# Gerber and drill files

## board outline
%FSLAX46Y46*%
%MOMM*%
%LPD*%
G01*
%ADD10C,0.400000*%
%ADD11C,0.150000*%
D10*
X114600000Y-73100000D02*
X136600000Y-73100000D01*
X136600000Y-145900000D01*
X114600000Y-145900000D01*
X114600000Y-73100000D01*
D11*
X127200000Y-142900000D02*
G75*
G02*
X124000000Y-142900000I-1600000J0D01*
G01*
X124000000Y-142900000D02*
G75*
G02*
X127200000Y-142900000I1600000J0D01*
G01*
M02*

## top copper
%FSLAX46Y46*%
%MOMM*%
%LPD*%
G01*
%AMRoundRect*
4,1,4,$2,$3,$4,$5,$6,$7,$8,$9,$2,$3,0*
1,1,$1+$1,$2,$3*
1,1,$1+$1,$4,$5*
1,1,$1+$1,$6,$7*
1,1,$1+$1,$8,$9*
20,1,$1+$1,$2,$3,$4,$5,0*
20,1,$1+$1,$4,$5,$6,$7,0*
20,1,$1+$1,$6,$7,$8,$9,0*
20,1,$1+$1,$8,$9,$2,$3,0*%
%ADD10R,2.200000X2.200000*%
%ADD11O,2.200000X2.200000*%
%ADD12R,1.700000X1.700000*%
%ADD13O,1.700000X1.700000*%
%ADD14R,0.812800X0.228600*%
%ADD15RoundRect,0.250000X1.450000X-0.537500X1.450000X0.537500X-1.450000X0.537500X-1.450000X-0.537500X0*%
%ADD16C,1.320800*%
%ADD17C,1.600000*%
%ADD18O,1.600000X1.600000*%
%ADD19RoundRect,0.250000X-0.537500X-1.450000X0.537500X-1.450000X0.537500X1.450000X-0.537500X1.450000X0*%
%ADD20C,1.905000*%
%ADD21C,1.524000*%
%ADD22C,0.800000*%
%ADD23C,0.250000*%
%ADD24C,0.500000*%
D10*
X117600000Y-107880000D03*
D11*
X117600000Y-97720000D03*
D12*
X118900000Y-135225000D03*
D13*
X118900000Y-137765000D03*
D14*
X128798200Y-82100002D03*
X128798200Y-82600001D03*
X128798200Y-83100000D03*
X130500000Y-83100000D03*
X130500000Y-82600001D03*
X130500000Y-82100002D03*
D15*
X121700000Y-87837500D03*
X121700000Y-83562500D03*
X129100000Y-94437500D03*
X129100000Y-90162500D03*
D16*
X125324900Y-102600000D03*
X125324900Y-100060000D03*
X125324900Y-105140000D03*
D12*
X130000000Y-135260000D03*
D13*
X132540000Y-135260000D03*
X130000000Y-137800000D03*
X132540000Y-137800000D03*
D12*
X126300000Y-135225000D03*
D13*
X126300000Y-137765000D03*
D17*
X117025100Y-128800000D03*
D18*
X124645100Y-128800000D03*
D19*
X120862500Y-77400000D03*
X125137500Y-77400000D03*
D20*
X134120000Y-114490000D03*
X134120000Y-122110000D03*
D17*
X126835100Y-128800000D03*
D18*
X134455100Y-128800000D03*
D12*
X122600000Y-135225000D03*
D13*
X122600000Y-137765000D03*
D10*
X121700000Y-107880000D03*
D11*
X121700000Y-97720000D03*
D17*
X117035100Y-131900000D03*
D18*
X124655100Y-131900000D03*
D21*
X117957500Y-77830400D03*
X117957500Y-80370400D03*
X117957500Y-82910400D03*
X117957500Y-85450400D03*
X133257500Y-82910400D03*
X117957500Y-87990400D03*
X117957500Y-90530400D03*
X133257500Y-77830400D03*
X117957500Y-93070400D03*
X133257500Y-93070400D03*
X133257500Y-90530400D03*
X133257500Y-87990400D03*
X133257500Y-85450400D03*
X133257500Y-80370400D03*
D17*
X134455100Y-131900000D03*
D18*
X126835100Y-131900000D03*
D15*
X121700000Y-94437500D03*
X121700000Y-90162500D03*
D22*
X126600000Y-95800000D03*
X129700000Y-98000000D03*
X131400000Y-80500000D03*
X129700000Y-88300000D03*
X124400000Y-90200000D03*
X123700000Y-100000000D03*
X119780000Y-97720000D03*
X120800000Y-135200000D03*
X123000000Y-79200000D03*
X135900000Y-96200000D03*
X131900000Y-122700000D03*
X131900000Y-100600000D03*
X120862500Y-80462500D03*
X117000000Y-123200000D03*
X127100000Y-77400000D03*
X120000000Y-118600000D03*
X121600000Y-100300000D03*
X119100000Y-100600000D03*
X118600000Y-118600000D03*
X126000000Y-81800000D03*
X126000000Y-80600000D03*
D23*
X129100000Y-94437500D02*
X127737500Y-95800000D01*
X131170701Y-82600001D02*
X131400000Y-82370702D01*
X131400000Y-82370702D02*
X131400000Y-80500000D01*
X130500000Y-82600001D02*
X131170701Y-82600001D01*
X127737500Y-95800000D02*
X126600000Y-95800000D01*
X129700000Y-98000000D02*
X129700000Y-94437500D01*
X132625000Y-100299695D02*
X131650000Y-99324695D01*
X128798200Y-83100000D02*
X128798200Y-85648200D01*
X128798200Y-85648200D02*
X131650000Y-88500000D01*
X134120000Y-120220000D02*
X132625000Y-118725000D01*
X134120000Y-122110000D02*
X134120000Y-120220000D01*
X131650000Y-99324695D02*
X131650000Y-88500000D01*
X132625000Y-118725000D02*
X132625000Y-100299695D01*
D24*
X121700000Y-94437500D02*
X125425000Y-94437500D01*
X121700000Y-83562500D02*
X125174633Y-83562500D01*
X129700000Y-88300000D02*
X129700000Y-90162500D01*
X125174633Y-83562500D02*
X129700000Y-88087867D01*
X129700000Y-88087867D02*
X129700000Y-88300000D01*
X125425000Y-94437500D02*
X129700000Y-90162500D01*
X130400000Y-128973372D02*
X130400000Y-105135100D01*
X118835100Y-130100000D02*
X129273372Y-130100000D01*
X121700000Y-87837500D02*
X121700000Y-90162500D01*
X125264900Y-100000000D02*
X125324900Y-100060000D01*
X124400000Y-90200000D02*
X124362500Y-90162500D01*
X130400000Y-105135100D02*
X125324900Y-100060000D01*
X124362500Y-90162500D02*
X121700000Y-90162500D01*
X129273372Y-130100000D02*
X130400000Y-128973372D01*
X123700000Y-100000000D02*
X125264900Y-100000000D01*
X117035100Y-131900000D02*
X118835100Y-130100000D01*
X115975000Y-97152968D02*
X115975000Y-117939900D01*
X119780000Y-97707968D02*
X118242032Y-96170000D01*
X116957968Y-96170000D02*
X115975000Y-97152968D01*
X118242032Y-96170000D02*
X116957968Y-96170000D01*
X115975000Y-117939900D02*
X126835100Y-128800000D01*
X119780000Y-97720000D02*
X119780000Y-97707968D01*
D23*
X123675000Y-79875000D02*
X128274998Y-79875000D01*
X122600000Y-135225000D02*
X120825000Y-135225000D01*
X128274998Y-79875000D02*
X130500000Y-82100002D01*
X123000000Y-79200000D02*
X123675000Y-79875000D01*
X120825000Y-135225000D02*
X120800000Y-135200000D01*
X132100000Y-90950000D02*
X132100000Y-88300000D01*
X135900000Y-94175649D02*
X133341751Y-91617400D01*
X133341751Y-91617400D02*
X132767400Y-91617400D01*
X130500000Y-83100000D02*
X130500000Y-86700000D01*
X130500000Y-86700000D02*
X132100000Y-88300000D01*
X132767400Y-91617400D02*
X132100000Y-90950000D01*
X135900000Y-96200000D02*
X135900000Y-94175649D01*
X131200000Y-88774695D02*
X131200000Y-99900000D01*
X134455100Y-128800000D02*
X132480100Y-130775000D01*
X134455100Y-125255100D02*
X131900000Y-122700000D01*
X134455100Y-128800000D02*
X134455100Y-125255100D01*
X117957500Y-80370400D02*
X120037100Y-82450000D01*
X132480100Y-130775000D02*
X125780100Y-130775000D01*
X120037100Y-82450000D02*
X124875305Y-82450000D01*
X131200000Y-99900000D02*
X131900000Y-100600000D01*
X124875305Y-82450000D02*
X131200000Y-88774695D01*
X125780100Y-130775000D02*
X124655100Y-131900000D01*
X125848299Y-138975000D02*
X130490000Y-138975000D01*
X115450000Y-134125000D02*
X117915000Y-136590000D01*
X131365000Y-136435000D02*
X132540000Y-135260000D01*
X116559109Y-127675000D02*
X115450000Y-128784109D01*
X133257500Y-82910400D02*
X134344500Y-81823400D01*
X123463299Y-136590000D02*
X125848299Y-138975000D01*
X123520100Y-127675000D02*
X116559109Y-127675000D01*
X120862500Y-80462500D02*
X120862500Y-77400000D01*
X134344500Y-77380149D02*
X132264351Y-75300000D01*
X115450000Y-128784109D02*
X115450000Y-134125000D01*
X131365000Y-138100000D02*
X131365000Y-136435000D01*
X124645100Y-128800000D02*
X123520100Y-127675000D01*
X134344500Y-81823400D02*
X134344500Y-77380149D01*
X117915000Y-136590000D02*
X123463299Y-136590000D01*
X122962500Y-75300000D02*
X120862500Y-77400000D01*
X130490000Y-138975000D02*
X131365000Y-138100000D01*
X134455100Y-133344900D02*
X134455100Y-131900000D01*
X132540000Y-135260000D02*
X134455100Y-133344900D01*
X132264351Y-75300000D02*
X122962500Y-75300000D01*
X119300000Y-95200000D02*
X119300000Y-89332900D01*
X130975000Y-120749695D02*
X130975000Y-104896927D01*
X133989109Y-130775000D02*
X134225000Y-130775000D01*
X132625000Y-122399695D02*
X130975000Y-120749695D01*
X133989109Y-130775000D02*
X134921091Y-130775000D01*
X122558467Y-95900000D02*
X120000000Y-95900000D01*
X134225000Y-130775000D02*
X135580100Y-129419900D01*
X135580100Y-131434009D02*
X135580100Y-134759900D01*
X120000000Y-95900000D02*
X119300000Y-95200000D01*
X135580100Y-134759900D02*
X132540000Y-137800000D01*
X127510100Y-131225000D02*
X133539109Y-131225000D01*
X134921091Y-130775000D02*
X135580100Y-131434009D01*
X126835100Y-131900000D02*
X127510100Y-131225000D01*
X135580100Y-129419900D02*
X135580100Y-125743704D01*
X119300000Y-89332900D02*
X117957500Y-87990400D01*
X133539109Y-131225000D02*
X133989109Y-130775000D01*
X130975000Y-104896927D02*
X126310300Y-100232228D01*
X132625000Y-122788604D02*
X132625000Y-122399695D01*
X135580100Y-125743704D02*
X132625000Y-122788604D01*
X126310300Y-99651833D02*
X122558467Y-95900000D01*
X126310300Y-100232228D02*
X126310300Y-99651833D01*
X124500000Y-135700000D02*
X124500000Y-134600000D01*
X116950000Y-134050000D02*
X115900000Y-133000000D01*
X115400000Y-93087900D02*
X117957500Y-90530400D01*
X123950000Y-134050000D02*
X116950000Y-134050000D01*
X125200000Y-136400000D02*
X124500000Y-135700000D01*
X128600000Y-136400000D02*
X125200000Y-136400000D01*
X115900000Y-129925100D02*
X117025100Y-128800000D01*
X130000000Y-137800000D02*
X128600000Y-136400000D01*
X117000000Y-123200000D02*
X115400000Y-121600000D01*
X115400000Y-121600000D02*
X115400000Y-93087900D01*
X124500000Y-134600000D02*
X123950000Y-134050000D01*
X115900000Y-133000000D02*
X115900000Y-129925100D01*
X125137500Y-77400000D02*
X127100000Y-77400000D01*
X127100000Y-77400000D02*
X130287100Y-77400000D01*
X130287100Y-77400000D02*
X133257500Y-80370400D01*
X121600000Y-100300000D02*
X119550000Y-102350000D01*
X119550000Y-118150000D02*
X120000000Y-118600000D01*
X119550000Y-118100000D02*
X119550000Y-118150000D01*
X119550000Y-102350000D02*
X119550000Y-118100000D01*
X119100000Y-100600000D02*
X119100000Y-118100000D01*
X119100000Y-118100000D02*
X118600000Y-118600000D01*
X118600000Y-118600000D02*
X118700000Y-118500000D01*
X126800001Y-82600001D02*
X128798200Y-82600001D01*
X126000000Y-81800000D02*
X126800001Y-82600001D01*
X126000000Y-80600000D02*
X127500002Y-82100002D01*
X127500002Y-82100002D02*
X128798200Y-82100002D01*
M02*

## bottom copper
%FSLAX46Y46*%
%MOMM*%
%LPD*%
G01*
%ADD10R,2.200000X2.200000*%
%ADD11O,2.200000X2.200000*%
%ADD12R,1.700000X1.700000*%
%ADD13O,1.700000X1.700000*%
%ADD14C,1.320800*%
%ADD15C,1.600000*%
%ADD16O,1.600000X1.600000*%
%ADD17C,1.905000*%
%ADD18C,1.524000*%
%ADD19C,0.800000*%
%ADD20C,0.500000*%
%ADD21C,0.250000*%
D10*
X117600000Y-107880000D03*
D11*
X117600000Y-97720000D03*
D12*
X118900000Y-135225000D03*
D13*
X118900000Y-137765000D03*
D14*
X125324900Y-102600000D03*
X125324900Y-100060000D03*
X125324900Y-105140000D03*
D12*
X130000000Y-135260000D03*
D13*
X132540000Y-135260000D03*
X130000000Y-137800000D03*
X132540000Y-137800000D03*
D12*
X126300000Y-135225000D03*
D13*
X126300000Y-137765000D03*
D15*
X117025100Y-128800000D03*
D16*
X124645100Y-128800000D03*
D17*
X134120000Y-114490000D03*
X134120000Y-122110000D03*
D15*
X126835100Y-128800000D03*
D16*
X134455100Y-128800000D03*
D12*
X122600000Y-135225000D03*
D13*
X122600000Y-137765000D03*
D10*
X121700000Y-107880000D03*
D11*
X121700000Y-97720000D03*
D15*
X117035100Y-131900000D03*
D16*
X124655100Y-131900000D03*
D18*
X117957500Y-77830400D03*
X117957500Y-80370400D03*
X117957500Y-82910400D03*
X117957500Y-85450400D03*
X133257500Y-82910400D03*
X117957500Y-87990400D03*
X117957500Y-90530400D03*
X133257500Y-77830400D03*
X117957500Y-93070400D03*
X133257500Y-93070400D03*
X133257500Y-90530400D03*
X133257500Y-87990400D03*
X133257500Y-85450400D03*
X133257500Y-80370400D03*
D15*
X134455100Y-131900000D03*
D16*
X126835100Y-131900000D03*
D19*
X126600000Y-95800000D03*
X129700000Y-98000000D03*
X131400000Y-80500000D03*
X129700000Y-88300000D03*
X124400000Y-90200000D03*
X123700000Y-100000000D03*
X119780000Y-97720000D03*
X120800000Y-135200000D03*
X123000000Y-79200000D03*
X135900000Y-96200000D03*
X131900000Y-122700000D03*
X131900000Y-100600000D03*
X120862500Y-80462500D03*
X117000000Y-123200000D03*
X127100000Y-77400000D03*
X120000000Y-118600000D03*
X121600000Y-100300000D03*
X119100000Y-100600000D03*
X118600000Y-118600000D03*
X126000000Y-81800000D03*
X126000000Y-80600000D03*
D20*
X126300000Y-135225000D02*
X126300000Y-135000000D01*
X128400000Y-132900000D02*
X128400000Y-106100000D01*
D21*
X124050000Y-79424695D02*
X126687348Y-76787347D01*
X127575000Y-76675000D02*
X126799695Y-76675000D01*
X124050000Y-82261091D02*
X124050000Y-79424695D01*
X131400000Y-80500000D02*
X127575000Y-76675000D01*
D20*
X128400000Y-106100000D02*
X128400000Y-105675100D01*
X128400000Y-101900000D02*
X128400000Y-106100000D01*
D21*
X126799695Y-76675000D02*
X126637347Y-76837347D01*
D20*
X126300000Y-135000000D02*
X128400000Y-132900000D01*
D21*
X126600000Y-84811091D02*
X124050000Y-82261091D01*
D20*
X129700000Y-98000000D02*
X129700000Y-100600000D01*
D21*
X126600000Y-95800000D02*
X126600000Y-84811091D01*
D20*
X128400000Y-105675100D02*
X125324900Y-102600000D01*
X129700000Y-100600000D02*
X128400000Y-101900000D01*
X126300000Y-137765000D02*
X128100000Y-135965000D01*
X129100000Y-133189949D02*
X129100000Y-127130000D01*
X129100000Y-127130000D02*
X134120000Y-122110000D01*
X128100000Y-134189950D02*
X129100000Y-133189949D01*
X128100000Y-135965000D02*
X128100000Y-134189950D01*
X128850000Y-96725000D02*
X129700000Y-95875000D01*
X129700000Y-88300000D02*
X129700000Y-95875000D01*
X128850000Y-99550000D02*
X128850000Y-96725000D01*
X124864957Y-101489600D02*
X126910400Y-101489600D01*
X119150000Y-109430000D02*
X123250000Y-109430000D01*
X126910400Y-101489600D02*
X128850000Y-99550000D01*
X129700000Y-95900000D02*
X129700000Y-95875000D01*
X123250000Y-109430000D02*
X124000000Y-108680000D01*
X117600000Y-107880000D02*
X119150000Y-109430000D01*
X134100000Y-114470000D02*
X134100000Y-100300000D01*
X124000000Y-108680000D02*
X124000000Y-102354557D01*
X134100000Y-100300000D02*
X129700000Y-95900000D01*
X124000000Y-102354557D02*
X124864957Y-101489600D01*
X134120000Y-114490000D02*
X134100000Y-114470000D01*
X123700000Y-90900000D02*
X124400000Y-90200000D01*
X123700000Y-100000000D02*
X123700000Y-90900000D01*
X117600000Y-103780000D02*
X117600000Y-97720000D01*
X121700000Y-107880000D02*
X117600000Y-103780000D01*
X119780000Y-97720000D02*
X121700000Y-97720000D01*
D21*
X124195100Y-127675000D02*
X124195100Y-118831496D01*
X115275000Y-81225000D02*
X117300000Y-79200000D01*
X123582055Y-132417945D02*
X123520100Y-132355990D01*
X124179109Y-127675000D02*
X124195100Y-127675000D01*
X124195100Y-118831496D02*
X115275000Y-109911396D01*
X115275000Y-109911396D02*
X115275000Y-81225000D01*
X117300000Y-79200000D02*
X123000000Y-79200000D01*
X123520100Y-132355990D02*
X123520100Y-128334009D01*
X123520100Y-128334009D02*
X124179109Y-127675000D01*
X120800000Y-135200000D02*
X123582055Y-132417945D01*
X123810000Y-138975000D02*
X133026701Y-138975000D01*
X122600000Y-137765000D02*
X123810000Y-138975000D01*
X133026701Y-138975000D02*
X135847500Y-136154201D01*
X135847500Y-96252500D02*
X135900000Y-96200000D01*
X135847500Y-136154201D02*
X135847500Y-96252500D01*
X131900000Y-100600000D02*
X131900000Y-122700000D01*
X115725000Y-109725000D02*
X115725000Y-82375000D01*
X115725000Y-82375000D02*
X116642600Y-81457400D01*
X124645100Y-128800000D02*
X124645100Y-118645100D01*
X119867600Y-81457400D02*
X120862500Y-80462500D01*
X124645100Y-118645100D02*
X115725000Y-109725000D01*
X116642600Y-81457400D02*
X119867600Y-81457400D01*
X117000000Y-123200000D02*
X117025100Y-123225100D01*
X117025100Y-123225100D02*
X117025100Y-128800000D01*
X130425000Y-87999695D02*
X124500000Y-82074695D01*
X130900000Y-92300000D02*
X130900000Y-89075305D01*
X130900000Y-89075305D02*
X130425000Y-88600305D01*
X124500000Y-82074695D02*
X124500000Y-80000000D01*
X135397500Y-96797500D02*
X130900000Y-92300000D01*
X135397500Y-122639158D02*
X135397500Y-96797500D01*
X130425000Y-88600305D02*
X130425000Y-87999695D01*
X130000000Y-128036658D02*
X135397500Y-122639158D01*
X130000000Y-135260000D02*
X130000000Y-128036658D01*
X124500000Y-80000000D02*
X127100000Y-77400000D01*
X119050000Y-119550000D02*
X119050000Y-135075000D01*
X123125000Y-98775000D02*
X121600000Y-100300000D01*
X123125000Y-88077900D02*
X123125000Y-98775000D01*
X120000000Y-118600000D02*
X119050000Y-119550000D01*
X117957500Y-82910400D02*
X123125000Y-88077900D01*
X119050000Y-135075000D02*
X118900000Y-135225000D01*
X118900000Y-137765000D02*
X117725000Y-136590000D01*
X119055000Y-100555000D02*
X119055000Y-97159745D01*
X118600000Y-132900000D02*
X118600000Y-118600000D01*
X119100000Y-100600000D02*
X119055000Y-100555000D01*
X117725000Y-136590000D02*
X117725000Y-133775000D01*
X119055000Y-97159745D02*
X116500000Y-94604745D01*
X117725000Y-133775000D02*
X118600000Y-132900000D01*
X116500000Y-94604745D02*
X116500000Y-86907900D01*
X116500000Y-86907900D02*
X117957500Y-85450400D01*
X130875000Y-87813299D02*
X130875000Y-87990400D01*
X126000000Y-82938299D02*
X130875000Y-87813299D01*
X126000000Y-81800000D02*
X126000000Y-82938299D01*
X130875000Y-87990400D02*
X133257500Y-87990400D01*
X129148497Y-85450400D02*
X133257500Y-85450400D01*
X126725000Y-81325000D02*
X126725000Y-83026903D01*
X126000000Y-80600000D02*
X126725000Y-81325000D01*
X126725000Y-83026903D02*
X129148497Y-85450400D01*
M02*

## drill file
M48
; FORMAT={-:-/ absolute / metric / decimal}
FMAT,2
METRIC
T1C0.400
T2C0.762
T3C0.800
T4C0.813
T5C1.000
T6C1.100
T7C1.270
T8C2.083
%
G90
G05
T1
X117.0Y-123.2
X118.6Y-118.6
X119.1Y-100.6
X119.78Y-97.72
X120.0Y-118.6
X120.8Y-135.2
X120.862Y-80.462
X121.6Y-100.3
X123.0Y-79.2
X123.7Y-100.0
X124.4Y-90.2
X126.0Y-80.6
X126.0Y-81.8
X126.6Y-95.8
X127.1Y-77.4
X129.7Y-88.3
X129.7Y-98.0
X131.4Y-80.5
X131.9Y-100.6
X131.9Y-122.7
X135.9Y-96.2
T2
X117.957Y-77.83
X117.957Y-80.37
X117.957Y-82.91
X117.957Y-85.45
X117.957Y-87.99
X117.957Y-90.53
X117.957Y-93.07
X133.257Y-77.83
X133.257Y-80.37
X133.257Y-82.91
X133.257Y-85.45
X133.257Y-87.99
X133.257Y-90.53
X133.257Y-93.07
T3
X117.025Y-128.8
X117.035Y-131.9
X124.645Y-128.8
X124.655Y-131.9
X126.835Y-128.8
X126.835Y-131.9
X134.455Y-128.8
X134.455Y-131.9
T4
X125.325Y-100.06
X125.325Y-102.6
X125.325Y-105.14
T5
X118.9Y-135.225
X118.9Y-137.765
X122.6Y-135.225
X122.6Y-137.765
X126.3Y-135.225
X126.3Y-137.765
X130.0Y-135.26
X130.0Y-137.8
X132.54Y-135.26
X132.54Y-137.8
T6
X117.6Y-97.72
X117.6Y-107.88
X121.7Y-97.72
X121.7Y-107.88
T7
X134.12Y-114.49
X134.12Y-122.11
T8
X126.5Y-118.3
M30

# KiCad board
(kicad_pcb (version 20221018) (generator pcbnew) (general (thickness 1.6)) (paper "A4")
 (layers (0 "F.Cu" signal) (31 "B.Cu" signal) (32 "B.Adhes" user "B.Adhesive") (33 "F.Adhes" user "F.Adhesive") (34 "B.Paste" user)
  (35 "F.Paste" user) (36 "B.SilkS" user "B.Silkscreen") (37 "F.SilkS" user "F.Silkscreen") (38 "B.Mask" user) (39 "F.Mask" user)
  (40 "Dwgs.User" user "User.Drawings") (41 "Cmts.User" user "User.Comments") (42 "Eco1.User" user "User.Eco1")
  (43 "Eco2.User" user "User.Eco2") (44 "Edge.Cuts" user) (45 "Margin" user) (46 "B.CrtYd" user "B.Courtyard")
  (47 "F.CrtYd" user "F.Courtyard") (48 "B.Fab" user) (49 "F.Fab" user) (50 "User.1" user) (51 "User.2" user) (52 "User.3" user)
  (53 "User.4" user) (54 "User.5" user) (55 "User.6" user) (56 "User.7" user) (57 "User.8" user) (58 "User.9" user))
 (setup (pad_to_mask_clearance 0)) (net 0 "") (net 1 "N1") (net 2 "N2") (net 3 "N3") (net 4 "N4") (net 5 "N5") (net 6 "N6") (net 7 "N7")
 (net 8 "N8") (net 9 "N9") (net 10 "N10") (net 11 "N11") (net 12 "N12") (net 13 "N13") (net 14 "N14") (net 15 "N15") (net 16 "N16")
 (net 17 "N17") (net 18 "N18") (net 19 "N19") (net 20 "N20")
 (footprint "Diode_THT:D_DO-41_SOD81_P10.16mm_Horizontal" (layer "F.Cu") (at 117.6 107.88 90)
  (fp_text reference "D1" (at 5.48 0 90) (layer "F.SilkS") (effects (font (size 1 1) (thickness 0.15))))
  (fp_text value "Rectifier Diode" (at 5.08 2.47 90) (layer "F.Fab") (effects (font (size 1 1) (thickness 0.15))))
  (pad "1" thru_hole rect (at 0 0 90) (size 2.2 2.2) (drill 1.1) (layers "*.Cu" "*.Mask") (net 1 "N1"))
  (pad "2" thru_hole oval (at 10.16 0 90) (size 2.2 2.2) (drill 1.1) (layers "*.Cu" "*.Mask") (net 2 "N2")))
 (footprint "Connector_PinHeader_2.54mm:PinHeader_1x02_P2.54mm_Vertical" (layer "F.Cu") (at 118.9 135.225)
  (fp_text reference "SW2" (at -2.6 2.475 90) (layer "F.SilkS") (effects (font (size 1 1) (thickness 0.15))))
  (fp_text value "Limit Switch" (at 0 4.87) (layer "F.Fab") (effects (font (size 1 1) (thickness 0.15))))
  (pad "1" thru_hole rect (at 0 0) (size 1.7 1.7) (drill 1) (layers "*.Cu" "*.Mask") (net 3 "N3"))
  (pad "2" thru_hole oval (at 0 2.54) (size 1.7 1.7) (drill 1) (layers "*.Cu" "*.Mask") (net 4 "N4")))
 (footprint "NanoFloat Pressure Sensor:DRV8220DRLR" (layer "F.Cu") (at 129.6491 82.600001)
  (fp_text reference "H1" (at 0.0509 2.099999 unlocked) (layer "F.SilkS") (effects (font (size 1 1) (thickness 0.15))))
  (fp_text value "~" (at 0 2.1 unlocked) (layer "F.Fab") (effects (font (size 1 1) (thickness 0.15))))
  (pad "1" smd rect (at -0.8509 -0.499999) (size 0.8128 0.2286) (layers "F.Cu" "F.Paste" "F.Mask") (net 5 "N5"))
  (pad "2" smd rect (at -0.8509 0) (size 0.8128 0.2286) (layers "F.Cu" "F.Paste" "F.Mask") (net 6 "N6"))
  (pad "3" smd rect (at -0.8509 0.499999) (size 0.8128 0.2286) (layers "F.Cu" "F.Paste" "F.Mask") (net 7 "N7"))
  (pad "4" smd rect (at 0.8509 0.499999) (size 0.8128 0.2286) (layers "F.Cu" "F.Paste" "F.Mask") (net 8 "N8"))
  (pad "5" smd rect (at 0.8509 0) (size 0.8128 0.2286) (layers "F.Cu" "F.Paste" "F.Mask") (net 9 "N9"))
  (pad "6" smd rect (at 0.8509 -0.499999) (size 0.8128 0.2286) (layers "F.Cu" "F.Paste" "F.Mask") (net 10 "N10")))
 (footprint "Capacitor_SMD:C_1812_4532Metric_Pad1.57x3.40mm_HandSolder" (layer "F.Cu") (at 121.7 85.7 90)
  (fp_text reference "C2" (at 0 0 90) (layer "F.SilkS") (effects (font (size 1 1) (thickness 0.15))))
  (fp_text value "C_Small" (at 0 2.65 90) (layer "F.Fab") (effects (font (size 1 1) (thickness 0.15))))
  (pad "1" smd roundrect (at -2.1375 0 90) (size 1.575 3.4) (layers "F.Cu" "F.Paste" "F.Mask") (roundrect_rratio 0.1587301587)
   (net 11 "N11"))
  (pad "2" smd roundrect (at 2.1375 0 90) (size 1.575 3.4) (layers "F.Cu" "F.Paste" "F.Mask") (roundrect_rratio 0.1587301587) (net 1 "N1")))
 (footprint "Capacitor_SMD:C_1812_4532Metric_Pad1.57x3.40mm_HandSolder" (layer "F.Cu") (at 129.1 92.3 90)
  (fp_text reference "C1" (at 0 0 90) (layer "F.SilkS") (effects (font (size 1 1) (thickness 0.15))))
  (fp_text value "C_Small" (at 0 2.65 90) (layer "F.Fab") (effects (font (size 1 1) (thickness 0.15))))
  (pad "1" smd roundrect (at -2.1375 0 90) (size 1.575 3.4) (layers "F.Cu" "F.Paste" "F.Mask") (roundrect_rratio 0.1587301587) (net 9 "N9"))
  (pad "2" smd roundrect (at 2.1375 0 90) (size 1.575 3.4) (layers "F.Cu" "F.Paste" "F.Mask") (roundrect_rratio 0.1587301587) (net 1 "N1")))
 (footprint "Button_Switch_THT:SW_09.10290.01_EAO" (layer "F.Cu") (at 125.3249 102.6 90)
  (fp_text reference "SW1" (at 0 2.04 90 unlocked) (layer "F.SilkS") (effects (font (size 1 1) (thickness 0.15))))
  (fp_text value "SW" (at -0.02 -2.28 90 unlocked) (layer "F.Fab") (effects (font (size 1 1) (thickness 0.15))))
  (pad "1" thru_hole circle (at 0 0 90) (size 1.3208 1.3208) (drill 0.8128) (layers "*.Cu" "*.Mask") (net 9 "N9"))
  (pad "2" thru_hole circle (at 2.54 0 90) (size 1.3208 1.3208) (drill 0.8128) (layers "*.Cu" "*.Mask") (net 11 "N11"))
  (pad "3" thru_hole circle (at -2.54 0 90) (size 1.3208 1.3208) (drill 0.8128) (layers "*.Cu" "*.Mask") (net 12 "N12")))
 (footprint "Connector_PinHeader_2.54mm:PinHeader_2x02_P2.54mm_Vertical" (layer "F.Cu") (at 130 135.26)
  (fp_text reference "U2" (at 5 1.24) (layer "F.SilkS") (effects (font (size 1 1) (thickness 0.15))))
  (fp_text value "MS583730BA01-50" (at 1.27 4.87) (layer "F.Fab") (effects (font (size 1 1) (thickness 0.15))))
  (pad "1" thru_hole rect (at 0 0) (size 1.7 1.7) (drill 1) (layers "*.Cu" "*.Mask") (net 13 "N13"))
  (pad "2" thru_hole oval (at 2.54 0) (size 1.7 1.7) (drill 1) (layers "*.Cu" "*.Mask") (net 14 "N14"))
  (pad "3" thru_hole oval (at 0 2.54) (size 1.7 1.7) (drill 1) (layers "*.Cu" "*.Mask") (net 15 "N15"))
  (pad "4" thru_hole oval (at 2.54 2.54) (size 1.7 1.7) (drill 1) (layers "*.Cu" "*.Mask") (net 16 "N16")))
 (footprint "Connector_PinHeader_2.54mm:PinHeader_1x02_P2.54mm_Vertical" (layer "F.Cu") (at 126.3 135.225)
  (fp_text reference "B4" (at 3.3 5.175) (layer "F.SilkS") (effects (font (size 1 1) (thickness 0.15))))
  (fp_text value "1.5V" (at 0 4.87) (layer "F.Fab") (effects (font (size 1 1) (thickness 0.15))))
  (pad "1" thru_hole rect (at 0 0) (size 1.7 1.7) (drill 1) (layers "*.Cu" "*.Mask") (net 9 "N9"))
  (pad "2" thru_hole oval (at 0 2.54) (size 1.7 1.7) (drill 1) (layers "*.Cu" "*.Mask") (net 7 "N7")))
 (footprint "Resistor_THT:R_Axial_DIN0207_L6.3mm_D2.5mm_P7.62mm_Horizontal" (layer "F.Cu") (at 117.0251 128.8)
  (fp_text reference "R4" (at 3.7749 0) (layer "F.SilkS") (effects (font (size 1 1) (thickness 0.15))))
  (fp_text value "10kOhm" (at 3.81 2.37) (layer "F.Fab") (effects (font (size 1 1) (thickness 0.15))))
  (pad "1" thru_hole circle (at 0 0) (size 1.6 1.6) (drill 0.8) (layers "*.Cu" "*.Mask") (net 15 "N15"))
  (pad "2" thru_hole oval (at 7.62 0) (size 1.6 1.6) (drill 0.8) (layers "*.Cu" "*.Mask") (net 14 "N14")))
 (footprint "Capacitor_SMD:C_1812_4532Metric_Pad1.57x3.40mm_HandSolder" (layer "F.Cu") (at 123 77.4)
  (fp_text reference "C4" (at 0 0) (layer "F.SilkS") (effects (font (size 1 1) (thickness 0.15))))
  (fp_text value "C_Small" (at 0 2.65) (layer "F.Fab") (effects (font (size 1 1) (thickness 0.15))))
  (pad "1" smd roundrect (at -2.1375 0) (size 1.575 3.4) (layers "F.Cu" "F.Paste" "F.Mask") (roundrect_rratio 0.1587301587) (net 14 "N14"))
  (pad "2" smd roundrect (at 2.1375 0) (size 1.575 3.4) (layers "F.Cu" "F.Paste" "F.Mask") (roundrect_rratio 0.1587301587) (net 13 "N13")))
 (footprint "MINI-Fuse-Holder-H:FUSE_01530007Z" (layer "F.Cu") (at 126.5 118.3 -90)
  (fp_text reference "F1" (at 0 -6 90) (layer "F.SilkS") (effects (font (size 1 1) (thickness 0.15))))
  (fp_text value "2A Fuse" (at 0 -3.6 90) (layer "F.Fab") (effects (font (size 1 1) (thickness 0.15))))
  (pad "" np_thru_hole circle (at 0 0 270) (size 2.0828 2.0828) (drill 2.0828) (layers "*.Cu" "*.Mask"))
  (pad "1" thru_hole circle (at -3.81 -7.62 270) (size 1.905 1.905) (drill 1.27) (layers "*.Cu" "*.Mask") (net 1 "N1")
   (solder_mask_margin 0.102))
  (pad "2" thru_hole circle (at 3.81 -7.62 270) (size 1.905 1.905) (drill 1.27) (layers "*.Cu" "*.Mask") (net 7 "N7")
   (solder_mask_margin 0.102)))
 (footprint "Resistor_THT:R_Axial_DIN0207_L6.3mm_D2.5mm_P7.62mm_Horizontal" (layer "F.Cu") (at 126.8351 128.8)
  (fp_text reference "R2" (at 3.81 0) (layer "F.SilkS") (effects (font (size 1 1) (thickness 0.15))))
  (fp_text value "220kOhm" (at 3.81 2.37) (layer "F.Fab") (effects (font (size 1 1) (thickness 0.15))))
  (pad "1" thru_hole circle (at 0 0) (size 1.6 1.6) (drill 0.8) (layers "*.Cu" "*.Mask") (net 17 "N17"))
  (pad "2" thru_hole oval (at 7.62 0) (size 1.6 1.6) (drill 0.8) (layers "*.Cu" "*.Mask") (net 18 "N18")))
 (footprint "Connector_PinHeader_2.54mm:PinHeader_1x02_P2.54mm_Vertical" (layer "F.Cu") (at 122.6 135.225)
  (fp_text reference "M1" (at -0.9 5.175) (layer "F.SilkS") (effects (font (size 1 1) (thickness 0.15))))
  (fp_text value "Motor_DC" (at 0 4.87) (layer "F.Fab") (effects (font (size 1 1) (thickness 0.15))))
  (pad "1" thru_hole rect (at 0 0) (size 1.7 1.7) (drill 1) (layers "*.Cu" "*.Mask") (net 10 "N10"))
  (pad "2" thru_hole oval (at 0 2.54) (size 1.7 1.7) (drill 1) (layers "*.Cu" "*.Mask") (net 8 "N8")))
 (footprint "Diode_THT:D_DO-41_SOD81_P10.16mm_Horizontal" (layer "F.Cu") (at 121.7 107.88 90)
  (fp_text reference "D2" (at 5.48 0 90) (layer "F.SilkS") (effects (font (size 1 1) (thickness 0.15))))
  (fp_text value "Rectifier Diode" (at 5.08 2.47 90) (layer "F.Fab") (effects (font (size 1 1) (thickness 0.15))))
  (pad "1" thru_hole rect (at 0 0 90) (size 2.2 2.2) (drill 1.1) (layers "*.Cu" "*.Mask") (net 2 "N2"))
  (pad "2" thru_hole oval (at 10.16 0 90) (size 2.2 2.2) (drill 1.1) (layers "*.Cu" "*.Mask") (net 17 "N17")))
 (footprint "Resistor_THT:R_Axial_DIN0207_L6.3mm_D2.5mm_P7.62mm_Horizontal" (layer "F.Cu") (at 117.0351 131.9)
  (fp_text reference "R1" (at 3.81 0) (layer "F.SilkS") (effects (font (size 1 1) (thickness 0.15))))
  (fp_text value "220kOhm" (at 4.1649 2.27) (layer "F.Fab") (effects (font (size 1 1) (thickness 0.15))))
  (pad "1" thru_hole circle (at 0 0) (size 1.6 1.6) (drill 0.8) (layers "*.Cu" "*.Mask") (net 11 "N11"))
  (pad "2" thru_hole oval (at 7.62 0) (size 1.6 1.6) (drill 0.8) (layers "*.Cu" "*.Mask") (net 18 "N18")))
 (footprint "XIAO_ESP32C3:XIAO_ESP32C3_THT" (layer "F.Cu") (at 125.5575 87.8704)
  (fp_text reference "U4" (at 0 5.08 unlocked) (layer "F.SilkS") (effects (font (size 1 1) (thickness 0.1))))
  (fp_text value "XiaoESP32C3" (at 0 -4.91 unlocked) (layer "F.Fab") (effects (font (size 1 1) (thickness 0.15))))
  (pad "0" thru_hole circle (at -7.6 -10.04) (size 1.524 1.524) (drill 0.762) (layers "*.Cu" "*.Mask"))
  (pad "1" thru_hole circle (at -7.6 -7.5) (size 1.524 1.524) (drill 0.762) (layers "*.Cu" "*.Mask") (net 18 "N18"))
  (pad "2" thru_hole circle (at -7.6 -4.96) (size 1.524 1.524) (drill 0.762) (layers "*.Cu" "*.Mask") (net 3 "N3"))
  (pad "3" thru_hole circle (at -7.6 -2.42) (size 1.524 1.524) (drill 0.762) (layers "*.Cu" "*.Mask") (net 4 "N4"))
  (pad "3V3" thru_hole circle (at 7.7 -4.96) (size 1.524 1.524) (drill 0.762) (layers "*.Cu" "*.Mask") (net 14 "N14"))
  (pad "4" thru_hole circle (at -7.6 0.12) (size 1.524 1.524) (drill 0.762) (layers "*.Cu" "*.Mask") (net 16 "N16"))
  (pad "5" thru_hole circle (at -7.6 2.66) (size 1.524 1.524) (drill 0.762) (layers "*.Cu" "*.Mask") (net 15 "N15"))
  (pad "5V" thru_hole circle (at 7.7 -10.04) (size 1.524 1.524) (drill 0.762) (layers "*.Cu" "*.Mask"))
  (pad "6" thru_hole circle (at -7.6 5.2) (size 1.524 1.524) (drill 0.762) (layers "*.Cu" "*.Mask"))
  (pad "7" thru_hole circle (at 7.7 5.2) (size 1.524 1.524) (drill 0.762) (layers "*.Cu" "*.Mask") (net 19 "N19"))
  (pad "8" thru_hole circle (at 7.7 2.66) (size 1.524 1.524) (drill 0.762) (layers "*.Cu" "*.Mask") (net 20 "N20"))
  (pad "9" thru_hole circle (at 7.7 0.12) (size 1.524 1.524) (drill 0.762) (layers "*.Cu" "*.Mask") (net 6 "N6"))
  (pad "10" thru_hole circle (at 7.7 -2.42) (size 1.524 1.524) (drill 0.762) (layers "*.Cu" "*.Mask") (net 5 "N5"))
  (pad "GND" thru_hole circle (at 7.7 -7.5) (size 1.524 1.524) (drill 0.762) (layers "*.Cu" "*.Mask") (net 13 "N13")))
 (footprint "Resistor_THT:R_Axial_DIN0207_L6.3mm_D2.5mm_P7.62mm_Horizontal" (layer "F.Cu") (at 134.4551 131.9 180)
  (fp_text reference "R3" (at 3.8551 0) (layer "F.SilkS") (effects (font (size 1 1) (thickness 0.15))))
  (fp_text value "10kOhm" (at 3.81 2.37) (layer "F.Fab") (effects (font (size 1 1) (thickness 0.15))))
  (pad "1" thru_hole circle (at 0 0 180) (size 1.6 1.6) (drill 0.8) (layers "*.Cu" "*.Mask") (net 14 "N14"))
  (pad "2" thru_hole oval (at 7.62 0 180) (size 1.6 1.6) (drill 0.8) (layers "*.Cu" "*.Mask") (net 16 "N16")))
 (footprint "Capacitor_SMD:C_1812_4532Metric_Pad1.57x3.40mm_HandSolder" (layer "F.Cu") (at 121.7 92.3 90)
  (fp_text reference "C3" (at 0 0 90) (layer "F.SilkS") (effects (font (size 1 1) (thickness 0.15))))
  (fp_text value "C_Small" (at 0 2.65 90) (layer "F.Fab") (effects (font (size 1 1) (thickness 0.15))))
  (pad "1" smd roundrect (at -2.1375 0 90) (size 1.575 3.4) (layers "F.Cu" "F.Paste" "F.Mask") (roundrect_rratio 0.1587301587) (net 1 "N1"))
  (pad "2" smd roundrect (at 2.1375 0 90) (size 1.575 3.4) (layers "F.Cu" "F.Paste" "F.Mask") (roundrect_rratio 0.1587301587) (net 11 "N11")))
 (gr_rect (start 114.6 73.1) (end 136.6 145.9) (stroke (width 0.4) (type default)) (fill none) (layer "Edge.Cuts"))
 (gr_circle (center 125.6 142.9) (end 127.2 142.9) (stroke (width 0.15) (type default)) (fill none) (layer "Edge.Cuts"))
 (segment (start 129.1 94.4375) (end 127.7375 95.8) (width 0.25) (layer "F.Cu") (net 9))
 (segment (start 131.170701 82.600001) (end 131.4 82.370702) (width 0.25) (layer "F.Cu") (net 9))
 (segment (start 131.4 82.370702) (end 131.4 80.5) (width 0.25) (layer "F.Cu") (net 9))
 (segment (start 130.5 82.600001) (end 131.170701 82.600001) (width 0.25) (layer "F.Cu") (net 9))
 (segment (start 127.7375 95.8) (end 126.6 95.8) (width 0.25) (layer "F.Cu") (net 9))
 (segment (start 129.7 98) (end 129.7 94.4375) (width 0.25) (layer "F.Cu") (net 9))
 (via (at 126.6 95.8) (size 0.8) (drill 0.4) (layers "F.Cu" "B.Cu") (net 9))
 (via (at 129.7 98) (size 0.8) (drill 0.4) (layers "F.Cu" "B.Cu") (free) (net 9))
 (via (at 131.4 80.5) (size 0.8) (drill 0.4) (layers "F.Cu" "B.Cu") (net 9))
 (segment (start 126.3 135.225) (end 126.3 135) (width 0.5) (layer "B.Cu") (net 9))
 (segment (start 128.4 132.9) (end 128.4 106.1) (width 0.5) (layer "B.Cu") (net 9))
 (segment (start 124.05 79.424695) (end 126.687348 76.787347) (width 0.25) (layer "B.Cu") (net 9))
 (segment (start 127.575 76.675) (end 126.799695 76.675) (width 0.25) (layer "B.Cu") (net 9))
 (segment (start 124.05 82.261091) (end 124.05 79.424695) (width 0.25) (layer "B.Cu") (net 9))
 (segment (start 131.4 80.5) (end 127.575 76.675) (width 0.25) (layer "B.Cu") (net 9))
 (segment (start 128.4 106.1) (end 128.4 105.6751) (width 0.5) (layer "B.Cu") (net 9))
 (segment (start 128.4 101.9) (end 128.4 106.1) (width 0.5) (layer "B.Cu") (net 9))
 (segment (start 126.799695 76.675) (end 126.637347 76.837347) (width 0.25) (layer "B.Cu") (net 9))
 (segment (start 126.3 135) (end 128.4 132.9) (width 0.5) (layer "B.Cu") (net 9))
 (segment (start 126.6 84.811091) (end 124.05 82.261091) (width 0.25) (layer "B.Cu") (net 9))
 (segment (start 129.7 98) (end 129.7 100.6) (width 0.5) (layer "B.Cu") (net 9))
 (segment (start 126.6 95.8) (end 126.6 84.811091) (width 0.25) (layer "B.Cu") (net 9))
 (segment (start 128.4 105.6751) (end 125.3249 102.6) (width 0.5) (layer "B.Cu") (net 9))
 (segment (start 129.7 100.6) (end 128.4 101.9) (width 0.5) (layer "B.Cu") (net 9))
 (segment (start 132.625 100.299695) (end 131.65 99.324695) (width 0.25) (layer "F.Cu") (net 7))
 (segment (start 128.7982 83.1) (end 128.7982 85.6482) (width 0.25) (layer "F.Cu") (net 7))
 (segment (start 128.7982 85.6482) (end 131.65 88.5) (width 0.25) (layer "F.Cu") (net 7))
 (segment (start 134.12 120.22) (end 132.625 118.725) (width 0.25) (layer "F.Cu") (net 7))
 (segment (start 134.12 122.11) (end 134.12 120.22) (width 0.25) (layer "F.Cu") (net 7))
 (segment (start 131.65 99.324695) (end 131.65 88.5) (width 0.25) (layer "F.Cu") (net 7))
 (segment (start 132.625 118.725) (end 132.625 100.299695) (width 0.25) (layer "F.Cu") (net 7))
 (segment (start 126.3 137.765) (end 128.1 135.965) (width 0.5) (layer "B.Cu") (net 7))
 (segment (start 129.1 133.189949) (end 129.1 127.13) (width 0.5) (layer "B.Cu") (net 7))
 (segment (start 129.1 127.13) (end 134.12 122.11) (width 0.5) (layer "B.Cu") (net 7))
 (segment (start 128.1 134.18995) (end 129.1 133.189949) (width 0.5) (layer "B.Cu") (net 7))
 (segment (start 128.1 135.965) (end 128.1 134.18995) (width 0.5) (layer "B.Cu") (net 7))
 (segment (start 121.7 94.4375) (end 125.425 94.4375) (width 0.5) (layer "F.Cu") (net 1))
 (segment (start 121.7 83.5625) (end 125.174633 83.5625) (width 0.5) (layer "F.Cu") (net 1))
 (segment (start 129.7 88.3) (end 129.7 90.1625) (width 0.5) (layer "F.Cu") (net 1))
 (segment (start 125.174633 83.5625) (end 129.7 88.087867) (width 0.5) (layer "F.Cu") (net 1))
 (segment (start 129.7 88.087867) (end 129.7 88.3) (width 0.5) (layer "F.Cu") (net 1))
 (segment (start 125.425 94.4375) (end 129.7 90.1625) (width 0.5) (layer "F.Cu") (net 1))
 (via (at 129.7 88.3) (size 0.8) (drill 0.4) (layers "F.Cu" "B.Cu") (free) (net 1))
 (segment (start 128.85 96.725) (end 129.7 95.875) (width 0.5) (layer "B.Cu") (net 1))
 (segment (start 129.7 88.3) (end 129.7 95.875) (width 0.5) (layer "B.Cu") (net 1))
 (segment (start 128.85 99.55) (end 128.85 96.725) (width 0.5) (layer "B.Cu") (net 1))
 (segment (start 124.864957 101.4896) (end 126.9104 101.4896) (width 0.5) (layer "B.Cu") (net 1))
 (segment (start 119.15 109.43) (end 123.25 109.43) (width 0.5) (layer "B.Cu") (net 1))
 (segment (start 126.9104 101.4896) (end 128.85 99.55) (width 0.5) (layer "B.Cu") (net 1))
 (segment (start 129.7 95.9) (end 129.7 95.875) (width 0.5) (layer "B.Cu") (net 1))
 (segment (start 123.25 109.43) (end 124 108.68) (width 0.5) (layer "B.Cu") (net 1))
 (segment (start 117.6 107.88) (end 119.15 109.43) (width 0.5) (layer "B.Cu") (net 1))
 (segment (start 134.1 114.47) (end 134.1 100.3) (width 0.5) (layer "B.Cu") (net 1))
 (segment (start 124 108.68) (end 124 102.354557) (width 0.5) (layer "B.Cu") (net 1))
 (segment (start 134.1 100.3) (end 129.7 95.9) (width 0.5) (layer "B.Cu") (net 1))
 (segment (start 124 102.354557) (end 124.864957 101.4896) (width 0.5) (layer "B.Cu") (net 1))
 (segment (start 134.12 114.49) (end 134.1 114.47) (width 0.5) (layer "B.Cu") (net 1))
 (segment (start 130.4 128.973372) (end 130.4 105.1351) (width 0.5) (layer "F.Cu") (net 11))
 (segment (start 118.8351 130.1) (end 129.273372 130.1) (width 0.5) (layer "F.Cu") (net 11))
 (segment (start 121.7 87.8375) (end 121.7 90.1625) (width 0.5) (layer "F.Cu") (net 11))
 (segment (start 125.2649 100) (end 125.3249 100.06) (width 0.5) (layer "F.Cu") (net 11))
 (segment (start 124.4 90.2) (end 124.3625 90.1625) (width 0.5) (layer "F.Cu") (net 11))
 (segment (start 130.4 105.1351) (end 125.3249 100.06) (width 0.5) (layer "F.Cu") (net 11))
 (segment (start 124.3625 90.1625) (end 121.7 90.1625) (width 0.5) (layer "F.Cu") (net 11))
 (segment (start 129.273372 130.1) (end 130.4 128.973372) (width 0.5) (layer "F.Cu") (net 11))
 (segment (start 123.7 100) (end 125.2649 100) (width 0.5) (layer "F.Cu") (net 11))
 (segment (start 117.0351 131.9) (end 118.8351 130.1) (width 0.5) (layer "F.Cu") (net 11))
 (via (at 124.4 90.2) (size 0.8) (drill 0.4) (layers "F.Cu" "B.Cu") (free) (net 11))
 (via (at 123.7 100) (size 0.8) (drill 0.4) (layers "F.Cu" "B.Cu") (free) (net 11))
 (segment (start 123.7 90.9) (end 124.4 90.2) (width 0.5) (layer "B.Cu") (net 11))
 (segment (start 123.7 100) (end 123.7 90.9) (width 0.5) (layer "B.Cu") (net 11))
 (segment (start 117.6 103.78) (end 117.6 97.72) (width 0.5) (layer "B.Cu") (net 2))
 (segment (start 121.7 107.88) (end 117.6 103.78) (width 0.5) (layer "B.Cu") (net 2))
 (segment (start 115.975 97.152968) (end 115.975 117.9399) (width 0.5) (layer "F.Cu") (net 17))
 (segment (start 119.78 97.707968) (end 118.242032 96.17) (width 0.5) (layer "F.Cu") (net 17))
 (segment (start 116.957968 96.17) (end 115.975 97.152968) (width 0.5) (layer "F.Cu") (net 17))
 (segment (start 118.242032 96.17) (end 116.957968 96.17) (width 0.5) (layer "F.Cu") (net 17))
 (segment (start 115.975 117.9399) (end 126.8351 128.8) (width 0.5) (layer "F.Cu") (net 17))
 (segment (start 119.78 97.72) (end 119.78 97.707968) (width 0.5) (layer "F.Cu") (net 17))
 (via (at 119.78 97.72) (size 0.8) (drill 0.4) (layers "F.Cu" "B.Cu") (free) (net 17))
 (segment (start 119.78 97.72) (end 121.7 97.72) (width 0.5) (layer "B.Cu") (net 17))
 (segment (start 123.675 79.875) (end 128.274998 79.875) (width 0.25) (layer "F.Cu") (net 10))
 (segment (start 122.6 135.225) (end 120.825 135.225) (width 0.25) (layer "F.Cu") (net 10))
 (segment (start 128.274998 79.875) (end 130.5 82.100002) (width 0.25) (layer "F.Cu") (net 10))
 (segment (start 123 79.2) (end 123.675 79.875) (width 0.25) (layer "F.Cu") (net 10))
 (segment (start 120.825 135.225) (end 120.8 135.2) (width 0.25) (layer "F.Cu") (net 10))
 (via (at 120.8 135.2) (size 0.8) (drill 0.4) (layers "F.Cu" "B.Cu") (free) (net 10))
 (via (at 123 79.2) (size 0.8) (drill 0.4) (layers "F.Cu" "B.Cu") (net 10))
 (segment (start 124.1951 127.675) (end 124.1951 118.831496) (width 0.25) (layer "B.Cu") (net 10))
 (segment (start 115.275 81.225) (end 117.3 79.2) (width 0.25) (layer "B.Cu") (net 10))
 (segment (start 123.582055 132.417945) (end 123.5201 132.35599) (width 0.25) (layer "B.Cu") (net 10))
 (segment (start 124.179109 127.675) (end 124.1951 127.675) (width 0.25) (layer "B.Cu") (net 10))
 (segment (start 124.1951 118.831496) (end 115.275 109.911396) (width 0.25) (layer "B.Cu") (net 10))
 (segment (start 115.275 109.911396) (end 115.275 81.225) (width 0.25) (layer "B.Cu") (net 10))
 (segment (start 117.3 79.2) (end 123 79.2) (width 0.25) (layer "B.Cu") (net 10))
 (segment (start 123.5201 132.35599) (end 123.5201 128.334009) (width 0.25) (layer "B.Cu") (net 10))
 (segment (start 123.5201 128.334009) (end 124.179109 127.675) (width 0.25) (layer "B.Cu") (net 10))
 (segment (start 120.8 135.2) (end 123.582055 132.417945) (width 0.25) (layer "B.Cu") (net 10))
 (segment (start 132.1 90.95) (end 132.1 88.3) (width 0.25) (layer "F.Cu") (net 8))
 (segment (start 135.9 94.175649) (end 133.341751 91.6174) (width 0.25) (layer "F.Cu") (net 8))
 (segment (start 133.341751 91.6174) (end 132.7674 91.6174) (width 0.25) (layer "F.Cu") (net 8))
 (segment (start 130.5 83.1) (end 130.5 86.7) (width 0.25) (layer "F.Cu") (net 8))
 (segment (start 130.5 86.7) (end 132.1 88.3) (width 0.25) (layer "F.Cu") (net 8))
 (segment (start 132.7674 91.6174) (end 132.1 90.95) (width 0.25) (layer "F.Cu") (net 8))
 (segment (start 135.9 96.2) (end 135.9 94.175649) (width 0.25) (layer "F.Cu") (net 8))
 (via (at 135.9 96.2) (size 0.8) (drill 0.4) (layers "F.Cu" "B.Cu") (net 8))
 (segment (start 123.81 138.975) (end 133.026701 138.975) (width 0.25) (layer "B.Cu") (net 8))
 (segment (start 122.6 137.765) (end 123.81 138.975) (width 0.25) (layer "B.Cu") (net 8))
 (segment (start 133.026701 138.975) (end 135.8475 136.154201) (width 0.25) (layer "B.Cu") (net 8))
 (segment (start 135.8475 96.2525) (end 135.9 96.2) (width 0.25) (layer "B.Cu") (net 8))
 (segment (start 135.8475 136.154201) (end 135.8475 96.2525) (width 0.25) (layer "B.Cu") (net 8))
 (segment (start 131.2 88.774695) (end 131.2 99.9) (width 0.25) (layer "F.Cu") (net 18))
 (segment (start 134.4551 128.8) (end 132.4801 130.775) (width 0.25) (layer "F.Cu") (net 18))
 (segment (start 134.4551 125.2551) (end 131.9 122.7) (width 0.25) (layer "F.Cu") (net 18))
 (segment (start 134.4551 128.8) (end 134.4551 125.2551) (width 0.25) (layer "F.Cu") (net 18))
 (segment (start 117.9575 80.3704) (end 120.0371 82.45) (width 0.25) (layer "F.Cu") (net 18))
 (segment (start 132.4801 130.775) (end 125.7801 130.775) (width 0.25) (layer "F.Cu") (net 18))
 (segment (start 120.0371 82.45) (end 124.875305 82.45) (width 0.25) (layer "F.Cu") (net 18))
 (segment (start 131.2 99.9) (end 131.9 100.6) (width 0.25) (layer "F.Cu") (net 18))
 (segment (start 124.875305 82.45) (end 131.2 88.774695) (width 0.25) (layer "F.Cu") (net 18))
 (segment (start 125.7801 130.775) (end 124.6551 131.9) (width 0.25) (layer "F.Cu") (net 18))
 (via (at 131.9 122.7) (size 0.8) (drill 0.4) (layers "F.Cu" "B.Cu") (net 18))
 (via (at 131.9 100.6) (size 0.8) (drill 0.4) (layers "F.Cu" "B.Cu") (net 18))
 (segment (start 131.9 100.6) (end 131.9 122.7) (width 0.25) (layer "B.Cu") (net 18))
 (segment (start 125.848299 138.975) (end 130.49 138.975) (width 0.25) (layer "F.Cu") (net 14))
 (segment (start 115.45 134.125) (end 117.915 136.59) (width 0.25) (layer "F.Cu") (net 14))
 (segment (start 131.365 136.435) (end 132.54 135.26) (width 0.25) (layer "F.Cu") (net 14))
 (segment (start 116.559109 127.675) (end 115.45 128.784109) (width 0.25) (layer "F.Cu") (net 14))
 (segment (start 133.2575 82.9104) (end 134.3445 81.8234) (width 0.25) (layer "F.Cu") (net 14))
 (segment (start 123.463299 136.59) (end 125.848299 138.975) (width 0.25) (layer "F.Cu") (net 14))
 (segment (start 123.5201 127.675) (end 116.559109 127.675) (width 0.25) (layer "F.Cu") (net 14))
 (segment (start 120.8625 80.4625) (end 120.8625 77.4) (width 0.25) (layer "F.Cu") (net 14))
 (segment (start 134.3445 77.380149) (end 132.264351 75.3) (width 0.25) (layer "F.Cu") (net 14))
 (segment (start 115.45 128.784109) (end 115.45 134.125) (width 0.25) (layer "F.Cu") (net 14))
 (segment (start 131.365 138.1) (end 131.365 136.435) (width 0.25) (layer "F.Cu") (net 14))
 (segment (start 124.6451 128.8) (end 123.5201 127.675) (width 0.25) (layer "F.Cu") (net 14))
 (segment (start 134.3445 81.8234) (end 134.3445 77.380149) (width 0.25) (layer "F.Cu") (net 14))
 (segment (start 117.915 136.59) (end 123.463299 136.59) (width 0.25) (layer "F.Cu") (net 14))
 (segment (start 122.9625 75.3) (end 120.8625 77.4) (width 0.25) (layer "F.Cu") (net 14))
 (segment (start 130.49 138.975) (end 131.365 138.1) (width 0.25) (layer "F.Cu") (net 14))
 (segment (start 134.4551 133.3449) (end 134.4551 131.9) (width 0.25) (layer "F.Cu") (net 14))
 (segment (start 132.54 135.26) (end 134.4551 133.3449) (width 0.25) (layer "F.Cu") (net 14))
 (segment (start 132.264351 75.3) (end 122.9625 75.3) (width 0.25) (layer "F.Cu") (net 14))
 (via (at 120.8625 80.4625) (size 0.8) (drill 0.4) (layers "F.Cu" "B.Cu") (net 14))
 (segment (start 115.725 109.725) (end 115.725 82.375) (width 0.25) (layer "B.Cu") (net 14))
 (segment (start 115.725 82.375) (end 116.6426 81.4574) (width 0.25) (layer "B.Cu") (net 14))
 (segment (start 124.6451 128.8) (end 124.6451 118.6451) (width 0.25) (layer "B.Cu") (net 14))
 (segment (start 119.8676 81.4574) (end 120.8625 80.4625) (width 0.25) (layer "B.Cu") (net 14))
 (segment (start 124.6451 118.6451) (end 115.725 109.725) (width 0.25) (layer "B.Cu") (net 14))
 (segment (start 116.6426 81.4574) (end 119.8676 81.4574) (width 0.25) (layer "B.Cu") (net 14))
 (segment (start 119.3 95.2) (end 119.3 89.3329) (width 0.25) (layer "F.Cu") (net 16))
 (segment (start 130.975 120.749695) (end 130.975 104.896927) (width 0.25) (layer "F.Cu") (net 16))
 (segment (start 133.989109 130.775) (end 134.225 130.775) (width 0.25) (layer "F.Cu") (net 16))
 (segment (start 132.625 122.399695) (end 130.975 120.749695) (width 0.25) (layer "F.Cu") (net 16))
 (segment (start 133.989109 130.775) (end 134.921091 130.775) (width 0.25) (layer "F.Cu") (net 16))
 (segment (start 122.558467 95.9) (end 120 95.9) (width 0.25) (layer "F.Cu") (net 16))
 (segment (start 134.225 130.775) (end 135.5801 129.4199) (width 0.25) (layer "F.Cu") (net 16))
 (segment (start 135.5801 131.434009) (end 135.5801 134.7599) (width 0.25) (layer "F.Cu") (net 16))
 (segment (start 120 95.9) (end 119.3 95.2) (width 0.25) (layer "F.Cu") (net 16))
 (segment (start 135.5801 134.7599) (end 132.54 137.8) (width 0.25) (layer "F.Cu") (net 16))
 (segment (start 127.5101 131.225) (end 133.539109 131.225) (width 0.25) (layer "F.Cu") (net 16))
 (segment (start 134.921091 130.775) (end 135.5801 131.434009) (width 0.25) (layer "F.Cu") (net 16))
 (segment (start 126.8351 131.9) (end 127.5101 131.225) (width 0.25) (layer "F.Cu") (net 16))
 (segment (start 135.5801 129.4199) (end 135.5801 125.743704) (width 0.25) (layer "F.Cu") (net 16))
 (segment (start 119.3 89.3329) (end 117.9575 87.9904) (width 0.25) (layer "F.Cu") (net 16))
 (segment (start 133.539109 131.225) (end 133.989109 130.775) (width 0.25) (layer "F.Cu") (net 16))
 (segment (start 130.975 104.896927) (end 126.3103 100.232228) (width 0.25) (layer "F.Cu") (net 16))
 (segment (start 132.625 122.788604) (end 132.625 122.399695) (width 0.25) (layer "F.Cu") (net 16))
 (segment (start 135.5801 125.743704) (end 132.625 122.788604) (width 0.25) (layer "F.Cu") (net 16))
 (segment (start 126.3103 99.651833) (end 122.558467 95.9) (width 0.25) (layer "F.Cu") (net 16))
 (segment (start 126.3103 100.232228) (end 126.3103 99.651833) (width 0.25) (layer "F.Cu") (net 16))
 (segment (start 124.5 135.7) (end 124.5 134.6) (width 0.25) (layer "F.Cu") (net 15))
 (segment (start 116.95 134.05) (end 115.9 133) (width 0.25) (layer "F.Cu") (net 15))
 (segment (start 115.4 93.0879) (end 117.9575 90.5304) (width 0.25) (layer "F.Cu") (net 15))
 (segment (start 123.95 134.05) (end 116.95 134.05) (width 0.25) (layer "F.Cu") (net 15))
 (segment (start 125.2 136.4) (end 124.5 135.7) (width 0.25) (layer "F.Cu") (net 15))
 (segment (start 128.6 136.4) (end 125.2 136.4) (width 0.25) (layer "F.Cu") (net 15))
 (segment (start 115.9 129.9251) (end 117.0251 128.8) (width 0.25) (layer "F.Cu") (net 15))
 (segment (start 130 137.8) (end 128.6 136.4) (width 0.25) (layer "F.Cu") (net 15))
 (segment (start 117 123.2) (end 115.4 121.6) (width 0.25) (layer "F.Cu") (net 15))
 (segment (start 115.4 121.6) (end 115.4 93.0879) (width 0.25) (layer "F.Cu") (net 15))
 (segment (start 124.5 134.6) (end 123.95 134.05) (width 0.25) (layer "F.Cu") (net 15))
 (segment (start 115.9 133) (end 115.9 129.9251) (width 0.25) (layer "F.Cu") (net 15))
 (via (at 117 123.2) (size 0.8) (drill 0.4) (layers "F.Cu" "B.Cu") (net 15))
 (segment (start 117 123.2) (end 117.0251 123.2251) (width 0.25) (layer "B.Cu") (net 15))
 (segment (start 117.0251 123.2251) (end 117.0251 128.8) (width 0.25) (layer "B.Cu") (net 15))
 (segment (start 125.1375 77.4) (end 127.1 77.4) (width 0.25) (layer "F.Cu") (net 13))
 (segment (start 127.1 77.4) (end 130.2871 77.4) (width 0.25) (layer "F.Cu") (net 13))
 (segment (start 130.2871 77.4) (end 133.2575 80.3704) (width 0.25) (layer "F.Cu") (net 13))
 (via (at 127.1 77.4) (size 0.8) (drill 0.4) (layers "F.Cu" "B.Cu") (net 13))
 (segment (start 130.425 87.999695) (end 124.5 82.074695) (width 0.25) (layer "B.Cu") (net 13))
 (segment (start 130.9 92.3) (end 130.9 89.075305) (width 0.25) (layer "B.Cu") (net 13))
 (segment (start 130.9 89.075305) (end 130.425 88.600305) (width 0.25) (layer "B.Cu") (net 13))
 (segment (start 124.5 82.074695) (end 124.5 80) (width 0.25) (layer "B.Cu") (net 13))
 (segment (start 135.3975 96.7975) (end 130.9 92.3) (width 0.25) (layer "B.Cu") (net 13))
 (segment (start 135.3975 122.639158) (end 135.3975 96.7975) (width 0.25) (layer "B.Cu") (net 13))
 (segment (start 130.425 88.600305) (end 130.425 87.999695) (width 0.25) (layer "B.Cu") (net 13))
 (segment (start 130 128.036658) (end 135.3975 122.639158) (width 0.25) (layer "B.Cu") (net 13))
 (segment (start 130 135.26) (end 130 128.036658) (width 0.25) (layer "B.Cu") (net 13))
 (segment (start 124.5 80) (end 127.1 77.4) (width 0.25) (layer "B.Cu") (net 13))
 (segment (start 121.6 100.3) (end 119.55 102.35) (width 0.25) (layer "F.Cu") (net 3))
 (segment (start 119.55 118.15) (end 120 118.6) (width 0.25) (layer "F.Cu") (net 3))
 (segment (start 119.55 118.1) (end 119.55 118.15) (width 0.25) (layer "F.Cu") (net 3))
 (segment (start 119.55 102.35) (end 119.55 118.1) (width 0.25) (layer "F.Cu") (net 3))
 (via (at 120 118.6) (size 0.8) (drill 0.4) (layers "F.Cu" "B.Cu") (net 3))
 (via (at 121.6 100.3) (size 0.8) (drill 0.4) (layers "F.Cu" "B.Cu") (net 3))
 (segment (start 119.05 119.55) (end 119.05 135.075) (width 0.25) (layer "B.Cu") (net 3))
 (segment (start 123.125 98.775) (end 121.6 100.3) (width 0.25) (layer "B.Cu") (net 3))
 (segment (start 123.125 88.0779) (end 123.125 98.775) (width 0.25) (layer "B.Cu") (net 3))
 (segment (start 120 118.6) (end 119.05 119.55) (width 0.25) (layer "B.Cu") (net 3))
 (segment (start 117.9575 82.9104) (end 123.125 88.0779) (width 0.25) (layer "B.Cu") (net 3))
 (segment (start 119.05 135.075) (end 118.9 135.225) (width 0.25) (layer "B.Cu") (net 3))
 (segment (start 119.1 100.6) (end 119.1 118.1) (width 0.25) (layer "F.Cu") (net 4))
 (segment (start 119.1 118.1) (end 118.6 118.6) (width 0.25) (layer "F.Cu") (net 4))
 (segment (start 118.6 118.6) (end 118.7 118.5) (width 0.25) (layer "F.Cu") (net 4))
 (via (at 119.1 100.6) (size 0.8) (drill 0.4) (layers "F.Cu" "B.Cu") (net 4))
 (via (at 118.6 118.6) (size 0.8) (drill 0.4) (layers "F.Cu" "B.Cu") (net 4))
 (segment (start 118.9 137.765) (end 117.725 136.59) (width 0.25) (layer "B.Cu") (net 4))
 (segment (start 119.055 100.555) (end 119.055 97.159745) (width 0.25) (layer "B.Cu") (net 4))
 (segment (start 118.6 132.9) (end 118.6 118.6) (width 0.25) (layer "B.Cu") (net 4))
 (segment (start 119.1 100.6) (end 119.055 100.555) (width 0.25) (layer "B.Cu") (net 4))
 (segment (start 117.725 136.59) (end 117.725 133.775) (width 0.25) (layer "B.Cu") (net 4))
 (segment (start 119.055 97.159745) (end 116.5 94.604745) (width 0.25) (layer "B.Cu") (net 4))
 (segment (start 117.725 133.775) (end 118.6 132.9) (width 0.25) (layer "B.Cu") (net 4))
 (segment (start 116.5 94.604745) (end 116.5 86.9079) (width 0.25) (layer "B.Cu") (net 4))
 (segment (start 116.5 86.9079) (end 117.9575 85.4504) (width 0.25) (layer "B.Cu") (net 4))
 (segment (start 126.800001 82.600001) (end 128.7982 82.600001) (width 0.25) (layer "F.Cu") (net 6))
 (segment (start 126 81.8) (end 126.800001 82.600001) (width 0.25) (layer "F.Cu") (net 6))
 (via (at 126 81.8) (size 0.8) (drill 0.4) (layers "F.Cu" "B.Cu") (free) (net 6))
 (segment (start 130.875 87.813299) (end 130.875 87.9904) (width 0.25) (layer "B.Cu") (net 6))
 (segment (start 126 82.938299) (end 130.875 87.813299) (width 0.25) (layer "B.Cu") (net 6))
 (segment (start 126 81.8) (end 126 82.938299) (width 0.25) (layer "B.Cu") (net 6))
 (segment (start 130.875 87.9904) (end 133.2575 87.9904) (width 0.25) (layer "B.Cu") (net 6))
 (segment (start 126 80.6) (end 127.500002 82.100002) (width 0.25) (layer "F.Cu") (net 5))
 (segment (start 127.500002 82.100002) (end 128.7982 82.100002) (width 0.25) (layer "F.Cu") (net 5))
 (via (at 126 80.6) (size 0.8) (drill 0.4) (layers "F.Cu" "B.Cu") (free) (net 5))
 (segment (start 129.148497 85.4504) (end 133.2575 85.4504) (width 0.25) (layer "B.Cu") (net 5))
 (segment (start 126.725 81.325) (end 126.725 83.026903) (width 0.25) (layer "B.Cu") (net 5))
 (segment (start 126 80.6) (end 126.725 81.325) (width 0.25) (layer "B.Cu") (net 5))
 (segment (start 126.725 83.026903) (end 129.148497 85.4504) (width 0.25) (layer "B.Cu") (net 5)))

